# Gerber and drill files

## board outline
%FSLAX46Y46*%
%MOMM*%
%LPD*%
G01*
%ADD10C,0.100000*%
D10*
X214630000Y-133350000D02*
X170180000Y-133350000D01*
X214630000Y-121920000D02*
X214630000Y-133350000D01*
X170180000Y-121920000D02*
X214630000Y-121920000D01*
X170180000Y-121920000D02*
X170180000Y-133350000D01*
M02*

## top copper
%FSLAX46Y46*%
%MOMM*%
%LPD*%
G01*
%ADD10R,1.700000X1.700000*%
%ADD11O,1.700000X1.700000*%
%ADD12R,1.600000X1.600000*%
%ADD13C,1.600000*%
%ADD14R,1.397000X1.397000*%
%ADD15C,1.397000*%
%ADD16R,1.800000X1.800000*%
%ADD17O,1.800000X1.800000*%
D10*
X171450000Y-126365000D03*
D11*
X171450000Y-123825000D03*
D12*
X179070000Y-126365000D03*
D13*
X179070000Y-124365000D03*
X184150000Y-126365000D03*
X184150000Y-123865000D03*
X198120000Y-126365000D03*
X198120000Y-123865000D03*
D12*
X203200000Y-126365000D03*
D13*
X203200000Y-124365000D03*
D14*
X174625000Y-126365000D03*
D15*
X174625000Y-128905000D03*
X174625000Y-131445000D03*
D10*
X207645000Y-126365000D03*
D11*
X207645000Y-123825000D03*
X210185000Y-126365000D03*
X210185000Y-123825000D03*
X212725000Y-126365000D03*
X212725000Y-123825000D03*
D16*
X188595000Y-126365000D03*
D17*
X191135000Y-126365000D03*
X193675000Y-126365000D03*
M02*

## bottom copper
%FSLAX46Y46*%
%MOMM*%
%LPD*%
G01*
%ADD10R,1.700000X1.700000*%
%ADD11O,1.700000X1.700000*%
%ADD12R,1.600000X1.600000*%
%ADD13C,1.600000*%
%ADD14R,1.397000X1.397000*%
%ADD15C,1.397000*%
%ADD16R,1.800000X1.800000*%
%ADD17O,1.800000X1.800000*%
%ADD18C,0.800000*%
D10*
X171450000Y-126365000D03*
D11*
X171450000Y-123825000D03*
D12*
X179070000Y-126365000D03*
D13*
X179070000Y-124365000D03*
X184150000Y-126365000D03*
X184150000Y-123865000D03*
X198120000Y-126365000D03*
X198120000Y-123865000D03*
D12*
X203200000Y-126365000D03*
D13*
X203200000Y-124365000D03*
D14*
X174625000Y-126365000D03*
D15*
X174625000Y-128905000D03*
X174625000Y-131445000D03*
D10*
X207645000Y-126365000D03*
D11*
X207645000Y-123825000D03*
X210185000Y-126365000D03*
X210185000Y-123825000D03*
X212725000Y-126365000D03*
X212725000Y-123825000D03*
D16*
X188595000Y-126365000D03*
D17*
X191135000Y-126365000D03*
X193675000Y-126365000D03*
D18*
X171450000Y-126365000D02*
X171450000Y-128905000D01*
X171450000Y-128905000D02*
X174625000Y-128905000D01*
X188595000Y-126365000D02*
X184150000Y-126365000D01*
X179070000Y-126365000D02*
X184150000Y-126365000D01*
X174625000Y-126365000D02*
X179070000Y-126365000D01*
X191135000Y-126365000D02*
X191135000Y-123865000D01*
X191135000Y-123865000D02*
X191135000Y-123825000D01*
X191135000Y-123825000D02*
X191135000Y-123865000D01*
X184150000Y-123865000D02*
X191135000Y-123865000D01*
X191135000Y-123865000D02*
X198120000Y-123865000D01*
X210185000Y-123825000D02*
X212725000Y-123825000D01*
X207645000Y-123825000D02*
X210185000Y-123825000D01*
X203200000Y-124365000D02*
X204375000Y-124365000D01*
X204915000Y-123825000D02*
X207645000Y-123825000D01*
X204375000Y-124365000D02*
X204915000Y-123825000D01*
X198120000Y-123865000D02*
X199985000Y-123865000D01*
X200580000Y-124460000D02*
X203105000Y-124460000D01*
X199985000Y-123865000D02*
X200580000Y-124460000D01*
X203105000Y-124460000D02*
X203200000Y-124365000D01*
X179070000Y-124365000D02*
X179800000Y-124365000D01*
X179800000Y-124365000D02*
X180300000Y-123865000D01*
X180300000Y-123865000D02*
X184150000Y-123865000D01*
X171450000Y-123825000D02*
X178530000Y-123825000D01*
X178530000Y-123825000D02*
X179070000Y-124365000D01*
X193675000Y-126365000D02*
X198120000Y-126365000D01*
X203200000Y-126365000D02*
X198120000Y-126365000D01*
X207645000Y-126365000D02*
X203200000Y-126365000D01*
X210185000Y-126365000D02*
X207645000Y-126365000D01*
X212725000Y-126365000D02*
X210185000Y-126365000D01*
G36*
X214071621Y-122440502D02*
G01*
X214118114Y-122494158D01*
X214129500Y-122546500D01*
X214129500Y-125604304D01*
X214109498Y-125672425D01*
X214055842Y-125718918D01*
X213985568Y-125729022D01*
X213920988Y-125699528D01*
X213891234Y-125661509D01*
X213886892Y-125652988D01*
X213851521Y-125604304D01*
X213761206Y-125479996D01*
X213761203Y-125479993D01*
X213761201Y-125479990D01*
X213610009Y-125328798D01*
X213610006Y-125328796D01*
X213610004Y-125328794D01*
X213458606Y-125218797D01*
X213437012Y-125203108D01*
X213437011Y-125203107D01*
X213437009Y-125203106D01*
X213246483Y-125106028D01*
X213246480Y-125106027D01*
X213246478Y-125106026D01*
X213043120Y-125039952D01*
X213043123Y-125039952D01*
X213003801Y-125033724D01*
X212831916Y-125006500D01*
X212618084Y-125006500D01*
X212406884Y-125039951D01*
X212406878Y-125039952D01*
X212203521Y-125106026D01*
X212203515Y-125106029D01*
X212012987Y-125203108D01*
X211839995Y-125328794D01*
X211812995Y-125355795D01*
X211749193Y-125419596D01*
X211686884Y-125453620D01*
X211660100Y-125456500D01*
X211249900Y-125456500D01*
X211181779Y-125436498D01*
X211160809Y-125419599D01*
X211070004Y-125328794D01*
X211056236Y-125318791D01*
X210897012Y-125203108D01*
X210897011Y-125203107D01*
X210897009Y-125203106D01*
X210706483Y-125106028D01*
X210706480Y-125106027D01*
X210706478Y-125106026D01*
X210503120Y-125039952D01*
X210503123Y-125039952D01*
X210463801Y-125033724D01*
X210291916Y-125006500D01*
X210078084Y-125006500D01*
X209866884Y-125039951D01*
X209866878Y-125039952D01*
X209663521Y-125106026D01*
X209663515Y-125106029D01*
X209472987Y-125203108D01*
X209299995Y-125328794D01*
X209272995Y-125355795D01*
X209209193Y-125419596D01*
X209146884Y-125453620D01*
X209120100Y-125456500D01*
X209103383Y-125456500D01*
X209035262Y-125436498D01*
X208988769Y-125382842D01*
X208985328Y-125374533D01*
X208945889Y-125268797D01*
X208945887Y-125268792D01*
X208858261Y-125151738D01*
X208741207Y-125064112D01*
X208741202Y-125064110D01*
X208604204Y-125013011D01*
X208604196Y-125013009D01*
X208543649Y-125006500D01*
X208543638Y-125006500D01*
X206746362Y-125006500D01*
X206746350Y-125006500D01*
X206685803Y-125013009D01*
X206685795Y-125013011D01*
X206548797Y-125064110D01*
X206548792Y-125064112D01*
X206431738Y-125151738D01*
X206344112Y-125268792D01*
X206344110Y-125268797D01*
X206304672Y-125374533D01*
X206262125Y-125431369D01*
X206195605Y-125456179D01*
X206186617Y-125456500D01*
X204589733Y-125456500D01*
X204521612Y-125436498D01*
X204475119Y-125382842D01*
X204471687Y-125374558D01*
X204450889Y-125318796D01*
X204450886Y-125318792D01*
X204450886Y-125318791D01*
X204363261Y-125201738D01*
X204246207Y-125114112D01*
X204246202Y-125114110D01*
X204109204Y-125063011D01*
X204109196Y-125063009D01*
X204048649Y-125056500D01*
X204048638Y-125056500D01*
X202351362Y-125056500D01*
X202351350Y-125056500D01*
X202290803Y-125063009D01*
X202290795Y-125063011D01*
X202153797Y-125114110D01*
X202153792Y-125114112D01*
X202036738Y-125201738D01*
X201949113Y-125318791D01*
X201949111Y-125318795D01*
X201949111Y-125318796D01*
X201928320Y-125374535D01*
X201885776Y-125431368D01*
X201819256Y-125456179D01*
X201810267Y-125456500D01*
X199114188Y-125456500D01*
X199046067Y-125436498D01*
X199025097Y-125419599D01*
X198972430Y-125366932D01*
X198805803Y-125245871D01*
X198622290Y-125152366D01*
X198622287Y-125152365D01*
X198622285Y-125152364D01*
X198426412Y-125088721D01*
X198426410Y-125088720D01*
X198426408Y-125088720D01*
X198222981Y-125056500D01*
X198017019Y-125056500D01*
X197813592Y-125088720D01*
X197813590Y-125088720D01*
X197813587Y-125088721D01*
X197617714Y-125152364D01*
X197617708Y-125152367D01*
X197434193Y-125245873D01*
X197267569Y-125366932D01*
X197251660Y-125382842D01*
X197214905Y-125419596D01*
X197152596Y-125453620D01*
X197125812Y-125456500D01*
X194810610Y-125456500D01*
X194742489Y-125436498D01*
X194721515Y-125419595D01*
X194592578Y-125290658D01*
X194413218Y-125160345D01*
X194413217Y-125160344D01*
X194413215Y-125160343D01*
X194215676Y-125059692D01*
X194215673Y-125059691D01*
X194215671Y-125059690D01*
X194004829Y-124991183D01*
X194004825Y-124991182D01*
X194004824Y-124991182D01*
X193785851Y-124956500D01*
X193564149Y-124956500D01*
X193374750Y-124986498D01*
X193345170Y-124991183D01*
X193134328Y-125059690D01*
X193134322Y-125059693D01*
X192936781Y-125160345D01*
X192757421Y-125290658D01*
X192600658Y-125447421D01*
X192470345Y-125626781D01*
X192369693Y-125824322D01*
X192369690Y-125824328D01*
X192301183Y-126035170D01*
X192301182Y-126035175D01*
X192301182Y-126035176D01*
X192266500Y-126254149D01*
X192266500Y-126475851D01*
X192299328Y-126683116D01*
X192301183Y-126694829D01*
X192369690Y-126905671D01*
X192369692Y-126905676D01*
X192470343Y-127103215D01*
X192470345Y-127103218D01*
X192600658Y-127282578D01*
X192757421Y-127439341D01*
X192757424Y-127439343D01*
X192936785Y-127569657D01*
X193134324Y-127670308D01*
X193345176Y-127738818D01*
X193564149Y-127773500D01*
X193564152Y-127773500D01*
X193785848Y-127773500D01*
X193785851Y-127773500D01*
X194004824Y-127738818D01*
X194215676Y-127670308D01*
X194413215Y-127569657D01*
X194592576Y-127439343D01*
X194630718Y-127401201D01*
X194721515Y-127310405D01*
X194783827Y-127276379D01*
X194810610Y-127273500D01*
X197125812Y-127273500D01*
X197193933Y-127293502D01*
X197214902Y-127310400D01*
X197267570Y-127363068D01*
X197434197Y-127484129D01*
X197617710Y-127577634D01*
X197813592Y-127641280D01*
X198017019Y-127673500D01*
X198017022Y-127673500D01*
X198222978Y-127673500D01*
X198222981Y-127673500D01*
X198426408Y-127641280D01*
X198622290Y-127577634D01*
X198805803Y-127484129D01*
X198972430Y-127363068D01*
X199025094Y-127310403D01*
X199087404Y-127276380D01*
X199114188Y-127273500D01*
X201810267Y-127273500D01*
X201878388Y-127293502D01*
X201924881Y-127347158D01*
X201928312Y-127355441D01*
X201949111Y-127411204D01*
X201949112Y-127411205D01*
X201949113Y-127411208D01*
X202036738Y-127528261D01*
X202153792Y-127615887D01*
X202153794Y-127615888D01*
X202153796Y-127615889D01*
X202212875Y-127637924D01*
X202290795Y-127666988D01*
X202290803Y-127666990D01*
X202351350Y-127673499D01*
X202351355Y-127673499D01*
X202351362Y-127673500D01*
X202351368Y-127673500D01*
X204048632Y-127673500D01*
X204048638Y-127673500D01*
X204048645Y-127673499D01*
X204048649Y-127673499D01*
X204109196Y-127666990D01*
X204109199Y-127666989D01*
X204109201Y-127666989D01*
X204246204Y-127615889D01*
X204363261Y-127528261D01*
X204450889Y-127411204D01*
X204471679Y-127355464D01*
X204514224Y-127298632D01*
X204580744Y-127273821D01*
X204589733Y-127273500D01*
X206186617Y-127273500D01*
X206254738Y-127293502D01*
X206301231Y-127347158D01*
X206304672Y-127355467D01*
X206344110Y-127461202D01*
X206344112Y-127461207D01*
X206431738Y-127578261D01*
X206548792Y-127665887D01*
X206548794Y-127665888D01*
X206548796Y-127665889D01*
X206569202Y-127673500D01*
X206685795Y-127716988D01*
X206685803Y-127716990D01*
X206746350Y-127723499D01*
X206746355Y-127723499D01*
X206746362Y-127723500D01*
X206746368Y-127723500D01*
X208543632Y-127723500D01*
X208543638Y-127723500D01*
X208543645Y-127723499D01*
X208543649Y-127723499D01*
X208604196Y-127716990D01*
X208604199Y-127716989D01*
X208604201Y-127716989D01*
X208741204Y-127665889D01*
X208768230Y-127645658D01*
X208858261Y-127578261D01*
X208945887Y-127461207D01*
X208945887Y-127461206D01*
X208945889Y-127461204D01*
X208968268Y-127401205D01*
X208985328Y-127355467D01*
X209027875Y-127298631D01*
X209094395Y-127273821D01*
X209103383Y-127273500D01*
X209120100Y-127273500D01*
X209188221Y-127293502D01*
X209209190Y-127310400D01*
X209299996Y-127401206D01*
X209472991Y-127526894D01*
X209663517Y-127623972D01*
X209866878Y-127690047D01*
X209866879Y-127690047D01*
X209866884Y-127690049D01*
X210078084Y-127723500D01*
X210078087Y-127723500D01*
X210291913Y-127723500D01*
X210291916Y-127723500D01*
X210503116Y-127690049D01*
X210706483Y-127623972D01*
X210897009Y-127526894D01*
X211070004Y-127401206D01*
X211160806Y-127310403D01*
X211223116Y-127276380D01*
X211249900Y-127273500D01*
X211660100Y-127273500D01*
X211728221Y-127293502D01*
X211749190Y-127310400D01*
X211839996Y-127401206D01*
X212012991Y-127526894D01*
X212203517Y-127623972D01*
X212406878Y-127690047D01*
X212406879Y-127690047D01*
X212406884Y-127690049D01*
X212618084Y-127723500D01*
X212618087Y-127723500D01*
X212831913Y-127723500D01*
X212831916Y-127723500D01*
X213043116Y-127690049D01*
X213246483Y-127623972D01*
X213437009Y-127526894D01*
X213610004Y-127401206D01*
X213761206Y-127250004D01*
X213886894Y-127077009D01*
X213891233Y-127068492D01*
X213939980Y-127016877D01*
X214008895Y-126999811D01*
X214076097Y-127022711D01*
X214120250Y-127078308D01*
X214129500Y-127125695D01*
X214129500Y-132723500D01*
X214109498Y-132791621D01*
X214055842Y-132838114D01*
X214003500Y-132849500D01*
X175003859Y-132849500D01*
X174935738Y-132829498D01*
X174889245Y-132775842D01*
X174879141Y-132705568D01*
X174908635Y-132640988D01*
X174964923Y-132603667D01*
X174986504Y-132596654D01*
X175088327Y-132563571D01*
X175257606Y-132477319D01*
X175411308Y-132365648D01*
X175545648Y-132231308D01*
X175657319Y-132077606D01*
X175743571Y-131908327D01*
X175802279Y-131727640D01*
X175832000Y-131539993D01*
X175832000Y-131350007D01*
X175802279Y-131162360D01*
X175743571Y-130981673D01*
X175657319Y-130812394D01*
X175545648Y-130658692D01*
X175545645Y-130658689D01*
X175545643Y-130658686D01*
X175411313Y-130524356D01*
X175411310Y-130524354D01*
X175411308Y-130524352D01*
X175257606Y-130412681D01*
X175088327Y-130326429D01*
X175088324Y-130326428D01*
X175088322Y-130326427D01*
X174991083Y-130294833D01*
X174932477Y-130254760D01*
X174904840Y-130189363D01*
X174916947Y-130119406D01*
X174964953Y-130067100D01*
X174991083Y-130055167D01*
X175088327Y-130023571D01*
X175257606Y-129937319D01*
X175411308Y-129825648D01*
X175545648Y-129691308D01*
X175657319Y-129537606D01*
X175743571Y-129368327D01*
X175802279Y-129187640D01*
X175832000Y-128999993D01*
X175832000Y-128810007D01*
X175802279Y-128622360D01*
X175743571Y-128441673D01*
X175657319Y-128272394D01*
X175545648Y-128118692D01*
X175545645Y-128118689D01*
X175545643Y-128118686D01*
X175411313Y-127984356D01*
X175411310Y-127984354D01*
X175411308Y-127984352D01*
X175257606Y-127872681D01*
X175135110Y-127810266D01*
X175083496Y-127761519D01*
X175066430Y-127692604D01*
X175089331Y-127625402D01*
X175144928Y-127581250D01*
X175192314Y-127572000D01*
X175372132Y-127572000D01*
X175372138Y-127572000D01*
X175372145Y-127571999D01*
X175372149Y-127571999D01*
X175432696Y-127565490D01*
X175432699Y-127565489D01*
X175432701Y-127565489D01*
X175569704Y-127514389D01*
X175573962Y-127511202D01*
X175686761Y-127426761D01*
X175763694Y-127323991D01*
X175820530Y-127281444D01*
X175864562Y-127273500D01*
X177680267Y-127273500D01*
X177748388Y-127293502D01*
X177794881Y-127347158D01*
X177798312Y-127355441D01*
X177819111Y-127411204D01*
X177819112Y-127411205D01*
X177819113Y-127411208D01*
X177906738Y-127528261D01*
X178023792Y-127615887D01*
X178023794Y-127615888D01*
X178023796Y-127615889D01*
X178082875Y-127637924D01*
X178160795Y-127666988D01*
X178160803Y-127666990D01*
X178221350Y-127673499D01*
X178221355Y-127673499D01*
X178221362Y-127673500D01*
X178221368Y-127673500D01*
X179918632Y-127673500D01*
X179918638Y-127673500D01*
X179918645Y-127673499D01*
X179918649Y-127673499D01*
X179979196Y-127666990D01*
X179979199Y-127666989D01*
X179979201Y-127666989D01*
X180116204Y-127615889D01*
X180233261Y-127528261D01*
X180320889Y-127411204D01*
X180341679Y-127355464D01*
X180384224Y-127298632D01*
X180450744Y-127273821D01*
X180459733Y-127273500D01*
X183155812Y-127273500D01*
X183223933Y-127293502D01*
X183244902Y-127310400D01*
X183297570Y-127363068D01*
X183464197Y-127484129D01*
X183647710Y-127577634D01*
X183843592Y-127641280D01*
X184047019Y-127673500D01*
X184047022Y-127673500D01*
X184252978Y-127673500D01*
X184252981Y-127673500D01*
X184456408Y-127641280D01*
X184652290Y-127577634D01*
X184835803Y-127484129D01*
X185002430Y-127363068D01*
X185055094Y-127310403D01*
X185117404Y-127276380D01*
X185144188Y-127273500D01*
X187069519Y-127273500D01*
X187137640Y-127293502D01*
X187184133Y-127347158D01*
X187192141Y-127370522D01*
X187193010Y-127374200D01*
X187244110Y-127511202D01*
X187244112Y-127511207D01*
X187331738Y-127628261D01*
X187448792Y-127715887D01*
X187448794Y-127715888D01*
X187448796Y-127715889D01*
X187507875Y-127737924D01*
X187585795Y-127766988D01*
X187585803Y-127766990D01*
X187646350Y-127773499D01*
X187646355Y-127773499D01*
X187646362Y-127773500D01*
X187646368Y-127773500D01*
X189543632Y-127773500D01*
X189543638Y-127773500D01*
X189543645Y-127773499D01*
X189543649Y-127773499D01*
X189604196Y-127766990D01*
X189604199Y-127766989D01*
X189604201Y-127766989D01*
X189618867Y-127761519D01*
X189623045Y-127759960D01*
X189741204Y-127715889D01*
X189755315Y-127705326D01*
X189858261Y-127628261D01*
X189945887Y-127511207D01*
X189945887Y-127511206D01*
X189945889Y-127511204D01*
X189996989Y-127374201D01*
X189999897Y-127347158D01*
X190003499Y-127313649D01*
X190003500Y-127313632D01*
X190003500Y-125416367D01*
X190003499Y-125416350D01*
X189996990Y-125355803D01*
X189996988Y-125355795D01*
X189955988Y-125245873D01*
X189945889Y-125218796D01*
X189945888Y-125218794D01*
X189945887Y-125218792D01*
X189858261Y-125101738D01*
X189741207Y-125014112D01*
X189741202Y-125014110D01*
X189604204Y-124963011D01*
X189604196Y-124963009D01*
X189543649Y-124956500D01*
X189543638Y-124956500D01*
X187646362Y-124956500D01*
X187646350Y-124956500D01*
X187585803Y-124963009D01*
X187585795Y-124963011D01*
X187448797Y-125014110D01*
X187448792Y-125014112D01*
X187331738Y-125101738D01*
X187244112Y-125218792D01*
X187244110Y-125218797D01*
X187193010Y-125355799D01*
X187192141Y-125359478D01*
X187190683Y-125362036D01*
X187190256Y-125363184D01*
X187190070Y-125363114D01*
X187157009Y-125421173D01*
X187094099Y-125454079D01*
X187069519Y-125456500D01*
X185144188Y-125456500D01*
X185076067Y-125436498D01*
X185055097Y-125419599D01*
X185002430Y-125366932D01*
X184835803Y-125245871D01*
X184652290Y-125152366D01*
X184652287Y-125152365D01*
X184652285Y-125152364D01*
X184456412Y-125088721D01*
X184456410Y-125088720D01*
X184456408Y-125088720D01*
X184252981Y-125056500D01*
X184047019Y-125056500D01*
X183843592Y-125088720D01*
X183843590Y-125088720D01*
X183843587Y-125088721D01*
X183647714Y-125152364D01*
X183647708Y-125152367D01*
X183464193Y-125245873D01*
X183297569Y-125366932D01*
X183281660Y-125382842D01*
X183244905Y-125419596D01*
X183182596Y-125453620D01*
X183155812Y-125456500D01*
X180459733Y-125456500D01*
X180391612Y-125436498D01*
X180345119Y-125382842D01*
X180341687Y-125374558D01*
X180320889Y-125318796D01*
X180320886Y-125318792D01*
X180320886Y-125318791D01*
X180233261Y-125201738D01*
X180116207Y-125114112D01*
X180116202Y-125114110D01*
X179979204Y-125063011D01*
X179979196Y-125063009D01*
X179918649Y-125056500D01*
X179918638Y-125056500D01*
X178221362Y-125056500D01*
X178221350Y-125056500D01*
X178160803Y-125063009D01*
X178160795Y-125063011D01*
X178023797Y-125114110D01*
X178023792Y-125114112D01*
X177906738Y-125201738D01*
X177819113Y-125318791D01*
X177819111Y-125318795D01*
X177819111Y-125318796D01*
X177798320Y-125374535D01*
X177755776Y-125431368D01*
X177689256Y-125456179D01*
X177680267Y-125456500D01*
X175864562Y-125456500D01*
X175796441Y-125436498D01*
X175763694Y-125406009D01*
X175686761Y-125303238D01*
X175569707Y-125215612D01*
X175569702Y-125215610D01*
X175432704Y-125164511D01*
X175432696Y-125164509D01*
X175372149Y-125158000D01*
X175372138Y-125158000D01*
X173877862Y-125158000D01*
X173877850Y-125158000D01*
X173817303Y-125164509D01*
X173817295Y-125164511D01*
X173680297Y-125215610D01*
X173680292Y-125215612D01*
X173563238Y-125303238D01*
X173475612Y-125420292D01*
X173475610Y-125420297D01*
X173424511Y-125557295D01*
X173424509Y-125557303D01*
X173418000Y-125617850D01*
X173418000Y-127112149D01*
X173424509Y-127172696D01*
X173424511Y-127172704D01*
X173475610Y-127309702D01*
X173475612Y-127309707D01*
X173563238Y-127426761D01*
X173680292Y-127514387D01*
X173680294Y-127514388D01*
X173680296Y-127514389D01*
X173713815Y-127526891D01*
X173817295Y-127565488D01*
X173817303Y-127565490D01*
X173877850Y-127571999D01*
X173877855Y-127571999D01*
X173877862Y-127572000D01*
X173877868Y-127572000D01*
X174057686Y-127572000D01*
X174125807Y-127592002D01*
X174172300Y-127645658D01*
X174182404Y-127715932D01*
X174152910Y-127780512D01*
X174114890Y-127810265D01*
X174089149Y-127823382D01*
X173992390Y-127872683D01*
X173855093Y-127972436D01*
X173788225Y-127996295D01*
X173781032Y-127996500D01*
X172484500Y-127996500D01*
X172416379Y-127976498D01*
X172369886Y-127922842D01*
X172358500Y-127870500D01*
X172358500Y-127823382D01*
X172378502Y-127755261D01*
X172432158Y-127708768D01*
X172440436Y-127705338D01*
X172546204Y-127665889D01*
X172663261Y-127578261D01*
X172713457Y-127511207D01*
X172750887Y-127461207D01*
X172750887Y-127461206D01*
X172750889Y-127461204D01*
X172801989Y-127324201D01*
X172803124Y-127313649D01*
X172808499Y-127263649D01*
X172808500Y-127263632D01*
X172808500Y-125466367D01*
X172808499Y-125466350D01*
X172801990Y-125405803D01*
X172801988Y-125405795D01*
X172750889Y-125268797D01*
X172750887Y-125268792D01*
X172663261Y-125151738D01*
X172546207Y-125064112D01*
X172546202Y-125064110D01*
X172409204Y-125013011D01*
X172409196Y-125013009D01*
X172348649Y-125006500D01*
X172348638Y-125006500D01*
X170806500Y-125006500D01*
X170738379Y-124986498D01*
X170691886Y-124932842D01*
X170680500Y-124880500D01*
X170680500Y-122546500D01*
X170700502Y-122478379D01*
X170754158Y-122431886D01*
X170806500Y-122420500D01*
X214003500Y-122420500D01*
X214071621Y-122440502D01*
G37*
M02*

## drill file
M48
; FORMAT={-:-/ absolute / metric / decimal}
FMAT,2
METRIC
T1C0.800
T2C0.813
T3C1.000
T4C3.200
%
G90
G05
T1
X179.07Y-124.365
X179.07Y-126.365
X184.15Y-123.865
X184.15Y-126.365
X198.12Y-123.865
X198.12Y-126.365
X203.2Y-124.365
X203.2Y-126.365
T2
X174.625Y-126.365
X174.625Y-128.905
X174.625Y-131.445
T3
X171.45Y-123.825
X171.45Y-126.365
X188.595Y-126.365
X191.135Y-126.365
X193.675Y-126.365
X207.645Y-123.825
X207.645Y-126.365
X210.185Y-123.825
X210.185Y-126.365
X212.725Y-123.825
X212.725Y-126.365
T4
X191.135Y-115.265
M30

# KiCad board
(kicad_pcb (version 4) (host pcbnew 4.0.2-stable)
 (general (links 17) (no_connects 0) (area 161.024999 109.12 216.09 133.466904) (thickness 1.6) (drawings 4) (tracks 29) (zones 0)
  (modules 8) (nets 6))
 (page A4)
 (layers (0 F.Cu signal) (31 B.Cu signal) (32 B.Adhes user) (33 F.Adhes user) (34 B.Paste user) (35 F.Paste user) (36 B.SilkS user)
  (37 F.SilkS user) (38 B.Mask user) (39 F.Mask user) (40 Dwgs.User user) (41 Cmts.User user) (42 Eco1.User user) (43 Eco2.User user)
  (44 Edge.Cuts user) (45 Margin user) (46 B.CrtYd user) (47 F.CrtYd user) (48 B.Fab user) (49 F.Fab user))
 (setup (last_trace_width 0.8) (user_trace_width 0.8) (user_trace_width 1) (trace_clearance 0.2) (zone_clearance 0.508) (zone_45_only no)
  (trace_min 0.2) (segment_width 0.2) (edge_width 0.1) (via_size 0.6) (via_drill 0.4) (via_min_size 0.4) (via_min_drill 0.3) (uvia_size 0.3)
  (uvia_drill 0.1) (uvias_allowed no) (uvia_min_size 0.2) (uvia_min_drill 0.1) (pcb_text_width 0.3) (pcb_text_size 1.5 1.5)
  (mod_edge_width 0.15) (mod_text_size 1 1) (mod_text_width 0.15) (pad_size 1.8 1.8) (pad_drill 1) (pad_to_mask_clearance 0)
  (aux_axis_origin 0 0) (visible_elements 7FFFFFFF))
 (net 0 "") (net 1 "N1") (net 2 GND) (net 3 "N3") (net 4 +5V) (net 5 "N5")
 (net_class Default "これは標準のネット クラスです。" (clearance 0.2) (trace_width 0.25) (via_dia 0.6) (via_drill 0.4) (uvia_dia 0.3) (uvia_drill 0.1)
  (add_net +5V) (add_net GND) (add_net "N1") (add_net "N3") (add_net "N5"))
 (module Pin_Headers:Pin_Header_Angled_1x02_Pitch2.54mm (layer F.Cu) (at 171.45 126.365 180)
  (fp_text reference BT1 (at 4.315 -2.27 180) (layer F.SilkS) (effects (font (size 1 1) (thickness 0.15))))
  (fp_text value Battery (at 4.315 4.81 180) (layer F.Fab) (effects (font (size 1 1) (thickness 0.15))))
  (pad 1 thru_hole rect (at 0 0 180) (size 1.7 1.7) (drill 1) (layers *.Cu *.Mask) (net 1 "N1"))
  (pad 2 thru_hole oval (at 0 2.54 180) (size 1.7 1.7) (drill 1) (layers *.Cu *.Mask) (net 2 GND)))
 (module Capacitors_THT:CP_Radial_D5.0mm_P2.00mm (layer F.Cu) (at 179.07 126.365 90)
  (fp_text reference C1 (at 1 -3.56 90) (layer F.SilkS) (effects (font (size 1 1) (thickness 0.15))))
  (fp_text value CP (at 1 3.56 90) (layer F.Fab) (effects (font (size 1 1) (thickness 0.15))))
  (pad 1 thru_hole rect (at 0 0 90) (size 1.6 1.6) (drill 0.8) (layers *.Cu *.Mask) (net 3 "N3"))
  (pad 2 thru_hole circle (at 2 0 90) (size 1.6 1.6) (drill 0.8) (layers *.Cu *.Mask) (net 2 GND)))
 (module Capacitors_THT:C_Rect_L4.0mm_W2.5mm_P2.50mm (layer F.Cu) (at 184.15 126.365 90)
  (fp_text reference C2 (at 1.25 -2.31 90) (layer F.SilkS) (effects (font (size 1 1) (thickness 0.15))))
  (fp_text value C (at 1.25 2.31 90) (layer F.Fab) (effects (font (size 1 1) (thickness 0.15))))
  (pad 1 thru_hole circle (at 0 0 90) (size 1.6 1.6) (drill 0.8) (layers *.Cu *.Mask) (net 3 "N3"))
  (pad 2 thru_hole circle (at 2.5 0 90) (size 1.6 1.6) (drill 0.8) (layers *.Cu *.Mask) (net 2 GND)))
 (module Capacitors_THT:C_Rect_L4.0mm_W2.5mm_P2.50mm (layer F.Cu) (at 198.12 126.365 90)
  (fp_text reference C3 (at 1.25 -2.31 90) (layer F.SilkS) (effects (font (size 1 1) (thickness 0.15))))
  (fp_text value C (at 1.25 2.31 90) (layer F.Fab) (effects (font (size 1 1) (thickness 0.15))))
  (pad 1 thru_hole circle (at 0 0 90) (size 1.6 1.6) (drill 0.8) (layers *.Cu *.Mask) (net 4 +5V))
  (pad 2 thru_hole circle (at 2.5 0 90) (size 1.6 1.6) (drill 0.8) (layers *.Cu *.Mask) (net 2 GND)))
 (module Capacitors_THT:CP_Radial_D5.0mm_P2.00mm (layer F.Cu) (at 203.2 126.365 90)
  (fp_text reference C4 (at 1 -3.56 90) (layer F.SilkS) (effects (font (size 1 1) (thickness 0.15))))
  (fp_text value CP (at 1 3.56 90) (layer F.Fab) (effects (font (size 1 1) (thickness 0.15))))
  (pad 1 thru_hole rect (at 0 0 90) (size 1.6 1.6) (drill 0.8) (layers *.Cu *.Mask) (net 4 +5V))
  (pad 2 thru_hole circle (at 2 0 90) (size 1.6 1.6) (drill 0.8) (layers *.Cu *.Mask) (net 2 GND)))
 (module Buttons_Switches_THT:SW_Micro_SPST (layer F.Cu) (at 174.625 128.905 270)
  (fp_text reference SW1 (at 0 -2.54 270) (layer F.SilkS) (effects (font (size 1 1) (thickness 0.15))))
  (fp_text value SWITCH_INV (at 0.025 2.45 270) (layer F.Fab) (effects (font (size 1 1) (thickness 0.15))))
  (pad 1 thru_hole rect (at -2.54 0 270) (size 1.397 1.397) (drill 0.8128) (layers *.Cu *.Mask) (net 3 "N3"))
  (pad 2 thru_hole circle (at 0 0 270) (size 1.397 1.397) (drill 0.8128) (layers *.Cu *.Mask) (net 1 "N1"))
  (pad 3 thru_hole circle (at 2.54 0 270) (size 1.397 1.397) (drill 0.8128) (layers *.Cu *.Mask) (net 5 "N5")))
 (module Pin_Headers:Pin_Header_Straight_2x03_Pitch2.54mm (layer F.Cu) (at 207.645 126.365 90)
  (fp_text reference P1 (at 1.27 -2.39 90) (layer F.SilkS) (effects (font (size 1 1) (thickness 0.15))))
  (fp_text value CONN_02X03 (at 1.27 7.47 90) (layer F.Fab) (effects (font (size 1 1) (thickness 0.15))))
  (pad 1 thru_hole rect (at 0 0 90) (size 1.7 1.7) (drill 1) (layers *.Cu *.Mask) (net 4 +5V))
  (pad 2 thru_hole oval (at 2.54 0 90) (size 1.7 1.7) (drill 1) (layers *.Cu *.Mask) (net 2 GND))
  (pad 3 thru_hole oval (at 0 2.54 90) (size 1.7 1.7) (drill 1) (layers *.Cu *.Mask) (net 4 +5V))
  (pad 4 thru_hole oval (at 2.54 2.54 90) (size 1.7 1.7) (drill 1) (layers *.Cu *.Mask) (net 2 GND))
  (pad 5 thru_hole oval (at 0 5.08 90) (size 1.7 1.7) (drill 1) (layers *.Cu *.Mask) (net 4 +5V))
  (pad 6 thru_hole oval (at 2.54 5.08 90) (size 1.7 1.7) (drill 1) (layers *.Cu *.Mask) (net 2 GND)))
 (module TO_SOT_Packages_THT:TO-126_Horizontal (layer F.Cu) (at 188.595 126.365)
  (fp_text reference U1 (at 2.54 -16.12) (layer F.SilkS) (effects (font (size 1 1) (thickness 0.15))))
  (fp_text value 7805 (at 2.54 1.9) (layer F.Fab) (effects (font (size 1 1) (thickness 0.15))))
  (pad None np_thru_hole oval (at 2.54 -11.1) (size 3.2 3.2) (drill 3.2) (layers *.Cu *.Mask))
  (pad 1 thru_hole rect (at 0 0) (size 1.8 1.8) (drill 1) (layers *.Cu *.Mask) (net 3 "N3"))
  (pad 2 thru_hole oval (at 2.54 0) (size 1.8 1.8) (drill 1) (layers *.Cu *.Mask) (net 2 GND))
  (pad 3 thru_hole oval (at 5.08 0) (size 1.8 1.8) (drill 1) (layers *.Cu *.Mask) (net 4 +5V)))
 (gr_line (start 214.63 133.35) (end 170.18 133.35) (angle 90) (layer Edge.Cuts) (width 0.1))
 (gr_line (start 214.63 121.92) (end 214.63 133.35) (angle 90) (layer Edge.Cuts) (width 0.1))
 (gr_line (start 170.18 121.92) (end 214.63 121.92) (angle 90) (layer Edge.Cuts) (width 0.1))
 (gr_line (start 170.18 121.92) (end 170.18 133.35) (angle 90) (layer Edge.Cuts) (width 0.1))
 (segment (start 171.45 126.365) (end 171.45 128.905) (width 0.8) (layer B.Cu) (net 1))
 (segment (start 171.45 128.905) (end 174.625 128.905) (width 0.8) (layer B.Cu) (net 1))
 (segment (start 188.595 126.365) (end 184.15 126.365) (width 0.8) (layer B.Cu) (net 3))
 (segment (start 179.07 126.365) (end 184.15 126.365) (width 0.8) (layer B.Cu) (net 3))
 (segment (start 174.625 126.365) (end 179.07 126.365) (width 0.8) (layer B.Cu) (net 3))
 (segment (start 191.135 126.365) (end 191.135 123.865) (width 0.8) (layer B.Cu) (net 2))
 (segment (start 191.135 123.865) (end 191.135 123.825) (width 0.8) (layer B.Cu) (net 2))
 (segment (start 191.135 123.825) (end 191.135 123.865) (width 0.8) (layer B.Cu) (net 2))
 (segment (start 184.15 123.865) (end 191.135 123.865) (width 0.8) (layer B.Cu) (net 2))
 (segment (start 191.135 123.865) (end 198.12 123.865) (width 0.8) (layer B.Cu) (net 2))
 (segment (start 210.185 123.825) (end 212.725 123.825) (width 0.8) (layer B.Cu) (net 2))
 (segment (start 207.645 123.825) (end 210.185 123.825) (width 0.8) (layer B.Cu) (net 2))
 (segment (start 203.2 124.365) (end 204.375 124.365) (width 0.8) (layer B.Cu) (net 2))
 (segment (start 204.915 123.825) (end 207.645 123.825) (width 0.8) (layer B.Cu) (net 2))
 (segment (start 204.375 124.365) (end 204.915 123.825) (width 0.8) (layer B.Cu) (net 2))
 (segment (start 198.12 123.865) (end 199.985 123.865) (width 0.8) (layer B.Cu) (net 2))
 (segment (start 200.58 124.46) (end 203.105 124.46) (width 0.8) (layer B.Cu) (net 2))
 (segment (start 199.985 123.865) (end 200.58 124.46) (width 0.8) (layer B.Cu) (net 2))
 (segment (start 203.105 124.46) (end 203.2 124.365) (width 0.8) (layer B.Cu) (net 2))
 (segment (start 179.07 124.365) (end 179.8 124.365) (width 0.8) (layer B.Cu) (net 2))
 (segment (start 179.8 124.365) (end 180.3 123.865) (width 0.8) (layer B.Cu) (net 2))
 (segment (start 180.3 123.865) (end 184.15 123.865) (width 0.8) (layer B.Cu) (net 2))
 (segment (start 171.45 123.825) (end 178.53 123.825) (width 0.8) (layer B.Cu) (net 2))
 (segment (start 178.53 123.825) (end 179.07 124.365) (width 0.8) (layer B.Cu) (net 2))
 (segment (start 193.675 126.365) (end 198.12 126.365) (width 0.8) (layer B.Cu) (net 4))
 (segment (start 203.2 126.365) (end 198.12 126.365) (width 0.8) (layer B.Cu) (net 4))
 (segment (start 207.645 126.365) (end 203.2 126.365) (width 0.8) (layer B.Cu) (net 4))
 (segment (start 210.185 126.365) (end 207.645 126.365) (width 0.8) (layer B.Cu) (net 4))
 (segment (start 212.725 126.365) (end 210.185 126.365) (width 0.8) (layer B.Cu) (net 4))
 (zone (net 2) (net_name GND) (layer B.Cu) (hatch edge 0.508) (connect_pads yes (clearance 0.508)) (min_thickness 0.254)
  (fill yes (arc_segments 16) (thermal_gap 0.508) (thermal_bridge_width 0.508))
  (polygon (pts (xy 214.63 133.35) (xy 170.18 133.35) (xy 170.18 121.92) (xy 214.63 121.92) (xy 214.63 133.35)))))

